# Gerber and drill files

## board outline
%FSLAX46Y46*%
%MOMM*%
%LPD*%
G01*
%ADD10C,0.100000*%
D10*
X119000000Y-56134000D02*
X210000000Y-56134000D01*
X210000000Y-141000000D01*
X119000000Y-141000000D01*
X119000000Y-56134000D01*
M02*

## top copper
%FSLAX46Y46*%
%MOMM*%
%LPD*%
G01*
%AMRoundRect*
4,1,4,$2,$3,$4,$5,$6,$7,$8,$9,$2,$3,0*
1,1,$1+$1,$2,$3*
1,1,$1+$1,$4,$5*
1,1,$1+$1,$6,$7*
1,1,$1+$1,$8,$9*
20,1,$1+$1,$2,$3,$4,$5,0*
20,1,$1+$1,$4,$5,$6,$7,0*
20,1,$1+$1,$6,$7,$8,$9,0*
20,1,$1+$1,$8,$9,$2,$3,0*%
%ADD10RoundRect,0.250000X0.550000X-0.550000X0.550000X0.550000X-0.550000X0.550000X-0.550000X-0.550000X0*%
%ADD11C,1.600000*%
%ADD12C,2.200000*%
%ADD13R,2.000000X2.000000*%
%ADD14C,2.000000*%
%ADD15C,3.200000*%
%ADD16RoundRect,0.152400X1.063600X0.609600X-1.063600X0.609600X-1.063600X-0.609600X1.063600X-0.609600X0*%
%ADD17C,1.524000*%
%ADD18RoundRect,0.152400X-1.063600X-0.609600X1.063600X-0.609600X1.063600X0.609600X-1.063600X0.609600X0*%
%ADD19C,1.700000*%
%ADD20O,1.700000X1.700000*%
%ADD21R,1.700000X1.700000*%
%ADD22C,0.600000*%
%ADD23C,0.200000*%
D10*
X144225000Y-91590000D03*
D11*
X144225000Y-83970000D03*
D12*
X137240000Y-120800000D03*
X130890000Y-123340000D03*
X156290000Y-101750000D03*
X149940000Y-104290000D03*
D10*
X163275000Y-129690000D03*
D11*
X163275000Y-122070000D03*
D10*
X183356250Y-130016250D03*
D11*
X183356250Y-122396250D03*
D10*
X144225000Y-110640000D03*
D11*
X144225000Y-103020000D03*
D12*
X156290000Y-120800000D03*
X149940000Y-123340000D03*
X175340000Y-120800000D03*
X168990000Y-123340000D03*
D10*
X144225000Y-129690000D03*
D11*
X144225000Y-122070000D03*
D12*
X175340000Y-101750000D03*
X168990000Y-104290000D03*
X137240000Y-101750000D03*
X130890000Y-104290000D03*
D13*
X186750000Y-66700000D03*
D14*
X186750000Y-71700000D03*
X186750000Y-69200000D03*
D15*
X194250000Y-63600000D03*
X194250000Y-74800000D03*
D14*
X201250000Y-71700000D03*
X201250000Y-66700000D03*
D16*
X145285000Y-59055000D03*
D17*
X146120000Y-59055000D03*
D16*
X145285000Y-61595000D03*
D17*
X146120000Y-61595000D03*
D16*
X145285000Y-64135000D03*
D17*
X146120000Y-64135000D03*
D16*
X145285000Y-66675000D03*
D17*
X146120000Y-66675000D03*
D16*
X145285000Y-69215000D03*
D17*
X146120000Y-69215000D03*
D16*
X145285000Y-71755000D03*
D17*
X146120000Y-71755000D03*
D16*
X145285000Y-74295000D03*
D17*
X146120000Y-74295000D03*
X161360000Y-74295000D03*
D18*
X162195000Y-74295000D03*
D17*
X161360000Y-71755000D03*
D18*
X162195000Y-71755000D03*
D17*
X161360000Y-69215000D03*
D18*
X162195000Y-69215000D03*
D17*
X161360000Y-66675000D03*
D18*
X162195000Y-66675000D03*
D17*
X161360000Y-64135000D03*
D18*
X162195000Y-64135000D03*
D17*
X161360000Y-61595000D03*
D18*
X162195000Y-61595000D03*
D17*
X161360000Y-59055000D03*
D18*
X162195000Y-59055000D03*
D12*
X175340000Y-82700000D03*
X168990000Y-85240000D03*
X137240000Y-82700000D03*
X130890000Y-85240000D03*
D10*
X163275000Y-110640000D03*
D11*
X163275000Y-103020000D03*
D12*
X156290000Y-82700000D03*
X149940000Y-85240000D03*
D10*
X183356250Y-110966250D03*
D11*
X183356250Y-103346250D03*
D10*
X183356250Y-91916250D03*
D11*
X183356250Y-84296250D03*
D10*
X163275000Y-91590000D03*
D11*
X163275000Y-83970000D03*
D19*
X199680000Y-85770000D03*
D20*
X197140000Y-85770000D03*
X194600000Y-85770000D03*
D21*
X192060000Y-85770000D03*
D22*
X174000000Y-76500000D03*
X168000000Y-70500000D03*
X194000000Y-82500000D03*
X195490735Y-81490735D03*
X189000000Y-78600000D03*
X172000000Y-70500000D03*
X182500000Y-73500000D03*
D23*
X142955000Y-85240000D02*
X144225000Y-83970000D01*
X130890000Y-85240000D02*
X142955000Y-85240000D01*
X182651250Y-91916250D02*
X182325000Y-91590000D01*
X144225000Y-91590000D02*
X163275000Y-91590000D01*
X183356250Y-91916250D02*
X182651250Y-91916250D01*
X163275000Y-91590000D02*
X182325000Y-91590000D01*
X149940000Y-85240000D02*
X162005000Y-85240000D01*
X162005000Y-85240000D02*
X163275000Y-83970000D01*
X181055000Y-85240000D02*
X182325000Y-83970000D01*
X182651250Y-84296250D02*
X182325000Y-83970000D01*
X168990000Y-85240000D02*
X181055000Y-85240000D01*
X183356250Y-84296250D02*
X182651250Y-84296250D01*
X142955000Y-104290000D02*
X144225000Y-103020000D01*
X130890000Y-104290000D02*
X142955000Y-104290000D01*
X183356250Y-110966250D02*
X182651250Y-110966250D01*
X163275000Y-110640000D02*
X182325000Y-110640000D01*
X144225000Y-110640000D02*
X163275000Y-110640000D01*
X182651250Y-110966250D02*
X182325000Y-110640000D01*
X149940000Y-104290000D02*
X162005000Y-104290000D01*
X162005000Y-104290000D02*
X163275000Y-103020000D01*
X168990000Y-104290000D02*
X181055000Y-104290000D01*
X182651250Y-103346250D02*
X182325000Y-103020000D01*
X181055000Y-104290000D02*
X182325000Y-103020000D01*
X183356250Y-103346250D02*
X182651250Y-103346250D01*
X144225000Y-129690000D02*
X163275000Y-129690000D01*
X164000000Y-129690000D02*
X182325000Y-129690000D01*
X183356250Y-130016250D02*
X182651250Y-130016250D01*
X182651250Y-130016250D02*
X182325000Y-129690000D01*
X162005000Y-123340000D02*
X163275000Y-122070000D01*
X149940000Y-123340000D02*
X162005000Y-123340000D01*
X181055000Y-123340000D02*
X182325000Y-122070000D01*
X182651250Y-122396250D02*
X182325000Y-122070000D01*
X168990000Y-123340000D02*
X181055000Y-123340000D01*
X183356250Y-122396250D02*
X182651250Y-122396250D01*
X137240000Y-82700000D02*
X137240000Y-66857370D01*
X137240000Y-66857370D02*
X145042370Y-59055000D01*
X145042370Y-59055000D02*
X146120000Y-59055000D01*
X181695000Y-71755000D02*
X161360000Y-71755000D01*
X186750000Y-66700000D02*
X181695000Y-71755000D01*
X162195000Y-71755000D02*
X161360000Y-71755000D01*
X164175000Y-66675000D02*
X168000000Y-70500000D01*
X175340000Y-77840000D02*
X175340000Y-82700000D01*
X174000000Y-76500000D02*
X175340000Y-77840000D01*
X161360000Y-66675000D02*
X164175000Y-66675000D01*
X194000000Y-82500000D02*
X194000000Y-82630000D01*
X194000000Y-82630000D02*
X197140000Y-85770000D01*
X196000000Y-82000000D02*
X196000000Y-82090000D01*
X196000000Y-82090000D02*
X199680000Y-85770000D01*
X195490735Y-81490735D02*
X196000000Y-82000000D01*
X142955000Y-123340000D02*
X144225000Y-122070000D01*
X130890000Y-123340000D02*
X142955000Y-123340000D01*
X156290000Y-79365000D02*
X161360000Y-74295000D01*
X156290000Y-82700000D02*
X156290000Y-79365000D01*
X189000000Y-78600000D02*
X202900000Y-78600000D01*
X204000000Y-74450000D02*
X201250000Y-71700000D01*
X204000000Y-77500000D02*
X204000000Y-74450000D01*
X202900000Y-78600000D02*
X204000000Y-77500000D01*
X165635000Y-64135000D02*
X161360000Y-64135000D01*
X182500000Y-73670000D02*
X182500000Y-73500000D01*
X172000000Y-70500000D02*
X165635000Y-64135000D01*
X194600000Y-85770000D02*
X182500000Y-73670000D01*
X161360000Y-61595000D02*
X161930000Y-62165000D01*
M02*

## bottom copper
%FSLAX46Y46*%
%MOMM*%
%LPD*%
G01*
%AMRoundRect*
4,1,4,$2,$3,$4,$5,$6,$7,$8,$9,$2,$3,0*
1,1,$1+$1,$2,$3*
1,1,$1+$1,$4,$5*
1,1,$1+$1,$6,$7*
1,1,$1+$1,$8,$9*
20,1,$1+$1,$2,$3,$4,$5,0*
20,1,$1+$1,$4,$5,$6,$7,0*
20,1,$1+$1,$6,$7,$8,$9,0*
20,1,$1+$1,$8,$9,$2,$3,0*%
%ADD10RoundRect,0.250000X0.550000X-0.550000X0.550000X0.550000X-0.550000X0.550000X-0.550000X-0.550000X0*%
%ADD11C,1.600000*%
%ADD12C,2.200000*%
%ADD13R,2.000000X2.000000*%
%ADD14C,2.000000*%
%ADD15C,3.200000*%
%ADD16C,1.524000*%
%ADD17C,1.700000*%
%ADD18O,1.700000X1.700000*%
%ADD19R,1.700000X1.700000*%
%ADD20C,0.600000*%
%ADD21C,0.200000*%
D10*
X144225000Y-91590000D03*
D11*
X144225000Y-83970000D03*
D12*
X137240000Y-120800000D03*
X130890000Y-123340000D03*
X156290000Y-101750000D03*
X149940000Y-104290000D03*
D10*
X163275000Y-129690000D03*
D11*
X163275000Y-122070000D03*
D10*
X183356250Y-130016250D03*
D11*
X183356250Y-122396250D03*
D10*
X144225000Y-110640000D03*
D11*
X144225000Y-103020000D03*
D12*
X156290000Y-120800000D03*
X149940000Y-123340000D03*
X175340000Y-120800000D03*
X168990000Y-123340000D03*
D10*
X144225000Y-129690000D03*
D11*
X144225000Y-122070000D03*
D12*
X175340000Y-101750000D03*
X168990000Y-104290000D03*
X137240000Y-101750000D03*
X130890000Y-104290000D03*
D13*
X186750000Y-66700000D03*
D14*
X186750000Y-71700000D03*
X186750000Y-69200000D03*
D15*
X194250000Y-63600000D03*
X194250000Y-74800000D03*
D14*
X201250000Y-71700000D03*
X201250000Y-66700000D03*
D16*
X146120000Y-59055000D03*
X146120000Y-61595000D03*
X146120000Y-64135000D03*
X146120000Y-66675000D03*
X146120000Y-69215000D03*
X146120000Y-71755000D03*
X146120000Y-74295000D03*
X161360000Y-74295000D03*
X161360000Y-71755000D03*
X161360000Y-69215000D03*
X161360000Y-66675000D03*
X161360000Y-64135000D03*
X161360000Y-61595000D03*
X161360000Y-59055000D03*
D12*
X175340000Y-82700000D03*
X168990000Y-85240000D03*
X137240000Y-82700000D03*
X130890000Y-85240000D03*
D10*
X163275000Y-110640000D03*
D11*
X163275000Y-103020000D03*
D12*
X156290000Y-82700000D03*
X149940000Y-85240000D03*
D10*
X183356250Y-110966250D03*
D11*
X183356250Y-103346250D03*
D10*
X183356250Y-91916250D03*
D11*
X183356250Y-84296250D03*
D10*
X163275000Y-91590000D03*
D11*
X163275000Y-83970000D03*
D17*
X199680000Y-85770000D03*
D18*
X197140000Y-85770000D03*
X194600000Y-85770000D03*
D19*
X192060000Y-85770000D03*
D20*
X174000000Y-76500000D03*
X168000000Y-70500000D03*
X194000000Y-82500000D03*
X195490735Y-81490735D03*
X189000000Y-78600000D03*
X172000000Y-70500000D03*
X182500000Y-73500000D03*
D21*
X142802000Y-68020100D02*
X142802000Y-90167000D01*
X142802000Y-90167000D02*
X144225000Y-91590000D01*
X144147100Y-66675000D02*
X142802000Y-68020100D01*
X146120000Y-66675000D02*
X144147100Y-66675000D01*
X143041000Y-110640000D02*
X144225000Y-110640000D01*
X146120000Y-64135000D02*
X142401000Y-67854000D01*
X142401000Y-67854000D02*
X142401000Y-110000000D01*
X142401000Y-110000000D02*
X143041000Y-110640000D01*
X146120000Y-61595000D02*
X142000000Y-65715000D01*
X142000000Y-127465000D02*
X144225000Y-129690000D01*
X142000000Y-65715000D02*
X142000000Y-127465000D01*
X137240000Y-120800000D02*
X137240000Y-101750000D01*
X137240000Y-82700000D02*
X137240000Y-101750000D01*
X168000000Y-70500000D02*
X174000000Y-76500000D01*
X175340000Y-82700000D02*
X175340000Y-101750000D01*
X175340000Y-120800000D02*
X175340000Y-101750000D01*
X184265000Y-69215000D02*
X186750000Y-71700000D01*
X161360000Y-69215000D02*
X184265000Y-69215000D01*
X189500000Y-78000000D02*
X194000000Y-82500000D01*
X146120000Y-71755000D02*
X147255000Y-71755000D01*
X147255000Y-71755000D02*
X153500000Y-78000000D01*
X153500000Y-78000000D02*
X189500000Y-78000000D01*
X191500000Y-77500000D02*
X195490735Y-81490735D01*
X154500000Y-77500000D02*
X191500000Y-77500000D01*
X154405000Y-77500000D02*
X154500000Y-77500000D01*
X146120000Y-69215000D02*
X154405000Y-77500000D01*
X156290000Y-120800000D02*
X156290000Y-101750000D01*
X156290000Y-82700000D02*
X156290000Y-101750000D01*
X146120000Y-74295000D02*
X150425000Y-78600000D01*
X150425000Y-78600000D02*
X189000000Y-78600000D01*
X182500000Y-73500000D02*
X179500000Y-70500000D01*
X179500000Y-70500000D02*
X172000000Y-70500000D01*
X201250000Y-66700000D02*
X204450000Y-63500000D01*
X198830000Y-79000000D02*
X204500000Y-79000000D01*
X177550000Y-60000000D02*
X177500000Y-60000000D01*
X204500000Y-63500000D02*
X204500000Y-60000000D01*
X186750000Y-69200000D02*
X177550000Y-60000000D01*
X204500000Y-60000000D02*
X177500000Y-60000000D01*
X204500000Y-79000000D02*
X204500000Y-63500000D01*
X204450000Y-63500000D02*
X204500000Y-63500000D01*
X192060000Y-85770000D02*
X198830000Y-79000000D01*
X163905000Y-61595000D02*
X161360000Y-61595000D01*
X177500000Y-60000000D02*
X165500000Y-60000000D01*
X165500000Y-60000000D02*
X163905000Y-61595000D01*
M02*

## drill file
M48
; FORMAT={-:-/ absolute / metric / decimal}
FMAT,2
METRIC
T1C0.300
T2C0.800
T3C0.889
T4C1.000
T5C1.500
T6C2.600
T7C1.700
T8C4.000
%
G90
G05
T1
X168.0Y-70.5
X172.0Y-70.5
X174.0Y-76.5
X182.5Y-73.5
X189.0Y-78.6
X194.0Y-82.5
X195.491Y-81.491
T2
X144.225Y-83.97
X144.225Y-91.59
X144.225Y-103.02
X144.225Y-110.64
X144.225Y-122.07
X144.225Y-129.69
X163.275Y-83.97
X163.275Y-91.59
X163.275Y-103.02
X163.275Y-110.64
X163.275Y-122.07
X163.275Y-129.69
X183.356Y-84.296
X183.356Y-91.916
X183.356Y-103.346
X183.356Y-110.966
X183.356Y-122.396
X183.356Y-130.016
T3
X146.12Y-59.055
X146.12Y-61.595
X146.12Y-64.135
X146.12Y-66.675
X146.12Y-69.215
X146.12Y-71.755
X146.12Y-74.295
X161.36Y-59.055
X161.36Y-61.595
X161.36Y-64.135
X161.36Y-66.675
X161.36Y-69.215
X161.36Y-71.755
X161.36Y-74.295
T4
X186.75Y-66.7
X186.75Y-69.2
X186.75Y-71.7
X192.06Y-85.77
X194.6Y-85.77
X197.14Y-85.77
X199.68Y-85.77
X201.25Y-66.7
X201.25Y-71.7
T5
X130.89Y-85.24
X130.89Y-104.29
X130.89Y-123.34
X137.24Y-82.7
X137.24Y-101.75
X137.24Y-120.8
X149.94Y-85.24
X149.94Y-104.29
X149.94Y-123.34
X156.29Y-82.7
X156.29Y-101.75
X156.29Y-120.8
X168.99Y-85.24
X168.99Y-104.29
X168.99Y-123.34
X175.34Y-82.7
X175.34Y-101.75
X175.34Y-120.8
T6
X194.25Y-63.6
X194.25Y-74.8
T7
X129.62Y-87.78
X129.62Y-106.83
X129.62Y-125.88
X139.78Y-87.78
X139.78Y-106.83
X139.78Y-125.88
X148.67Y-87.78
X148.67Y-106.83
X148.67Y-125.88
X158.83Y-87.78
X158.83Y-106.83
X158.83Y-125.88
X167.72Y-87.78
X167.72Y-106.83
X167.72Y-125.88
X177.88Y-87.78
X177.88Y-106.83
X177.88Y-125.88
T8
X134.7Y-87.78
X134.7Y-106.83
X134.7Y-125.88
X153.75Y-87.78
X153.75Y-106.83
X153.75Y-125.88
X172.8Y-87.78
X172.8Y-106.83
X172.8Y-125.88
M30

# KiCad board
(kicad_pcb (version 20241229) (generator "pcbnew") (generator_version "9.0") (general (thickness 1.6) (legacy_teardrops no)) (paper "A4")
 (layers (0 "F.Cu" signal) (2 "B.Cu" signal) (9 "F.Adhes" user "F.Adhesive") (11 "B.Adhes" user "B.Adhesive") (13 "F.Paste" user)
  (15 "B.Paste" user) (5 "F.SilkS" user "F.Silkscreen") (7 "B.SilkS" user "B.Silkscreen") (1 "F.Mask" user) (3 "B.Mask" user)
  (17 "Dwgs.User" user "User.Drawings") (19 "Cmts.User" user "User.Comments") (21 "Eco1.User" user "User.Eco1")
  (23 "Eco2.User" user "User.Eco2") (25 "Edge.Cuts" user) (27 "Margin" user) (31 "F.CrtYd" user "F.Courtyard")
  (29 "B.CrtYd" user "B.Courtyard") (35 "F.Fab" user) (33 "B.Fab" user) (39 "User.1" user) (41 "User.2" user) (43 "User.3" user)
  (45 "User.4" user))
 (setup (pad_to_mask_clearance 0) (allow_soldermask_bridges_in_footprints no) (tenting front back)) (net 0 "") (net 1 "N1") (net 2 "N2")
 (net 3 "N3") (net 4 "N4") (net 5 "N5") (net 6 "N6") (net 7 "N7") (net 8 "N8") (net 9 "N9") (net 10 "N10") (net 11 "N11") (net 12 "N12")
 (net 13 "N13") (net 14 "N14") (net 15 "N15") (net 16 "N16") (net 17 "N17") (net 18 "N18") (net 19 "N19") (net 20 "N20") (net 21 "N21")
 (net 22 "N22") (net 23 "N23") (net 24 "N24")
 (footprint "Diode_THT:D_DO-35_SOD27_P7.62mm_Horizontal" (layer "F.Cu") (at 144.225 91.59 90)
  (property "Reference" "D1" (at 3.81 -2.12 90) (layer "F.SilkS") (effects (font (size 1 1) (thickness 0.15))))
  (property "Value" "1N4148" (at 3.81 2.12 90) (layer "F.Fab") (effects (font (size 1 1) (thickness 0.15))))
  (pad "1" thru_hole roundrect (at 0 0 90) (size 1.6 1.6) (drill 0.8) (layers "*.Cu" "*.Mask") (remove_unused_layers no)
   (roundrect_rratio 0.15625) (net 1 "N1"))
  (pad "2" thru_hole circle (at 7.62 0 90) (size 1.6 1.6) (drill 0.8) (layers "*.Cu" "*.Mask") (remove_unused_layers no) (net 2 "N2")))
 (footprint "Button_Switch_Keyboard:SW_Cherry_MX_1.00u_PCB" (layer "F.Cu") (at 137.24 120.8)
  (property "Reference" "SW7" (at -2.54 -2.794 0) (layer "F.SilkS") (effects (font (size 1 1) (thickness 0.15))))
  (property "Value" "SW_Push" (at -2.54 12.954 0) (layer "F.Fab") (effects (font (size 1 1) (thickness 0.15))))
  (pad "" np_thru_hole circle (at -7.62 5.08) (size 1.7 1.7) (drill 1.7) (layers "*.Cu" "*.Mask"))
  (pad "" np_thru_hole circle (at -2.54 5.08) (size 4 4) (drill 4) (layers "*.Cu" "*.Mask"))
  (pad "" np_thru_hole circle (at 2.54 5.08) (size 1.7 1.7) (drill 1.7) (layers "*.Cu" "*.Mask"))
  (pad "1" thru_hole circle (at 0 0) (size 2.2 2.2) (drill 1.5) (layers "*.Cu" "*.Mask") (remove_unused_layers no) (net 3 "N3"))
  (pad "2" thru_hole circle (at -6.35 2.54) (size 2.2 2.2) (drill 1.5) (layers "*.Cu" "*.Mask") (remove_unused_layers no) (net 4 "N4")))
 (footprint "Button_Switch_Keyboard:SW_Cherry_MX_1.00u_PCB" (layer "F.Cu") (at 156.29 101.75)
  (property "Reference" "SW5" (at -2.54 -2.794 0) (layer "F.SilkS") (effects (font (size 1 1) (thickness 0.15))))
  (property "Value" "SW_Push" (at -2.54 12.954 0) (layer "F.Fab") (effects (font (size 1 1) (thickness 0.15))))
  (pad "" np_thru_hole circle (at -7.62 5.08) (size 1.7 1.7) (drill 1.7) (layers "*.Cu" "*.Mask"))
  (pad "" np_thru_hole circle (at -2.54 5.08) (size 4 4) (drill 4) (layers "*.Cu" "*.Mask"))
  (pad "" np_thru_hole circle (at 2.54 5.08) (size 1.7 1.7) (drill 1.7) (layers "*.Cu" "*.Mask"))
  (pad "1" thru_hole circle (at 0 0) (size 2.2 2.2) (drill 1.5) (layers "*.Cu" "*.Mask") (remove_unused_layers no) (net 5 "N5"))
  (pad "2" thru_hole circle (at -6.35 2.54) (size 2.2 2.2) (drill 1.5) (layers "*.Cu" "*.Mask") (remove_unused_layers no) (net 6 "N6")))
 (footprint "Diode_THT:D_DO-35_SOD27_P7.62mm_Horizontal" (layer "F.Cu") (at 163.275 129.69 90)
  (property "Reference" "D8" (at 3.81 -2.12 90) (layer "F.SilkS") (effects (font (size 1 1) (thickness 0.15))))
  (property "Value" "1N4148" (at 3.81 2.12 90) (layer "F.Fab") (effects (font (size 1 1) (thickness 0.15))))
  (pad "1" thru_hole roundrect (at 0 0 90) (size 1.6 1.6) (drill 0.8) (layers "*.Cu" "*.Mask") (remove_unused_layers no)
   (roundrect_rratio 0.15625) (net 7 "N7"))
  (pad "2" thru_hole circle (at 7.62 0 90) (size 1.6 1.6) (drill 0.8) (layers "*.Cu" "*.Mask") (remove_unused_layers no) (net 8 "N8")))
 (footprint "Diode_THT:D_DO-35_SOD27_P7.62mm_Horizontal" (layer "F.Cu") (at 183.35625 130.01625 90)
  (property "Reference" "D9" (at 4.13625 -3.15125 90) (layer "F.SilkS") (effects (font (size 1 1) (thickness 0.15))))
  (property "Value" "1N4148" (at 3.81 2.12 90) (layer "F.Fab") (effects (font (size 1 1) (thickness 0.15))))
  (pad "1" thru_hole roundrect (at 0 0 90) (size 1.6 1.6) (drill 0.8) (layers "*.Cu" "*.Mask") (remove_unused_layers no)
   (roundrect_rratio 0.15625) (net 7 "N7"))
  (pad "2" thru_hole circle (at 7.62 0 90) (size 1.6 1.6) (drill 0.8) (layers "*.Cu" "*.Mask") (remove_unused_layers no) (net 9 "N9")))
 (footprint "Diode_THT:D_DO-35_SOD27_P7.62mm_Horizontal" (layer "F.Cu") (at 144.225 110.64 90)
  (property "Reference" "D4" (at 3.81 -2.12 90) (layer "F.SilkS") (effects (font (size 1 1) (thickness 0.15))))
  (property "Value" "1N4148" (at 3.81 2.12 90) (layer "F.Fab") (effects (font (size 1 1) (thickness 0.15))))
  (pad "1" thru_hole roundrect (at 0 0 90) (size 1.6 1.6) (drill 0.8) (layers "*.Cu" "*.Mask") (remove_unused_layers no)
   (roundrect_rratio 0.15625) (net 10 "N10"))
  (pad "2" thru_hole circle (at 7.62 0 90) (size 1.6 1.6) (drill 0.8) (layers "*.Cu" "*.Mask") (remove_unused_layers no) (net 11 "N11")))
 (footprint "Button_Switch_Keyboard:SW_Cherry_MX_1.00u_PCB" (layer "F.Cu") (at 156.29 120.8)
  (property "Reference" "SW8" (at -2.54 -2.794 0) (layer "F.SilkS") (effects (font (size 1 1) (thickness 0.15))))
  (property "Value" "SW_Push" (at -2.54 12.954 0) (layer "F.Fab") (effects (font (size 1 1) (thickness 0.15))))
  (pad "" np_thru_hole circle (at -7.62 5.08) (size 1.7 1.7) (drill 1.7) (layers "*.Cu" "*.Mask"))
  (pad "" np_thru_hole circle (at -2.54 5.08) (size 4 4) (drill 4) (layers "*.Cu" "*.Mask"))
  (pad "" np_thru_hole circle (at 2.54 5.08) (size 1.7 1.7) (drill 1.7) (layers "*.Cu" "*.Mask"))
  (pad "1" thru_hole circle (at 0 0) (size 2.2 2.2) (drill 1.5) (layers "*.Cu" "*.Mask") (remove_unused_layers no) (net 5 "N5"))
  (pad "2" thru_hole circle (at -6.35 2.54) (size 2.2 2.2) (drill 1.5) (layers "*.Cu" "*.Mask") (remove_unused_layers no) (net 8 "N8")))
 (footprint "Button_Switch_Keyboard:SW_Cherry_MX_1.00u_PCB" (layer "F.Cu") (at 175.34 120.8)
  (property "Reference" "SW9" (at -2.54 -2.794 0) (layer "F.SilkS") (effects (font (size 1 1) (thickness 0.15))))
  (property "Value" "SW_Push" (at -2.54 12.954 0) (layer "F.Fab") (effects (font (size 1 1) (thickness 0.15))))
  (pad "" np_thru_hole circle (at -7.62 5.08) (size 1.7 1.7) (drill 1.7) (layers "*.Cu" "*.Mask"))
  (pad "" np_thru_hole circle (at -2.54 5.08) (size 4 4) (drill 4) (layers "*.Cu" "*.Mask"))
  (pad "" np_thru_hole circle (at 2.54 5.08) (size 1.7 1.7) (drill 1.7) (layers "*.Cu" "*.Mask"))
  (pad "1" thru_hole circle (at 0 0) (size 2.2 2.2) (drill 1.5) (layers "*.Cu" "*.Mask") (remove_unused_layers no) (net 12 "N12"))
  (pad "2" thru_hole circle (at -6.35 2.54) (size 2.2 2.2) (drill 1.5) (layers "*.Cu" "*.Mask") (remove_unused_layers no) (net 9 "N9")))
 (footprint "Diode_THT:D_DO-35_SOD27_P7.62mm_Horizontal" (layer "F.Cu") (at 144.225 129.69 90)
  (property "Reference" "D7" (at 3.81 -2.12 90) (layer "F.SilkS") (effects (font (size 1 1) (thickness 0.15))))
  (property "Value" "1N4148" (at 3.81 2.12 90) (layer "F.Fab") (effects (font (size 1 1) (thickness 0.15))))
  (pad "1" thru_hole roundrect (at 0 0 90) (size 1.6 1.6) (drill 0.8) (layers "*.Cu" "*.Mask") (remove_unused_layers no)
   (roundrect_rratio 0.15625) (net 7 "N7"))
  (pad "2" thru_hole circle (at 7.62 0 90) (size 1.6 1.6) (drill 0.8) (layers "*.Cu" "*.Mask") (remove_unused_layers no) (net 4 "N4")))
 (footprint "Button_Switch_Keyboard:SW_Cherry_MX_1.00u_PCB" (layer "F.Cu") (at 175.34 101.75)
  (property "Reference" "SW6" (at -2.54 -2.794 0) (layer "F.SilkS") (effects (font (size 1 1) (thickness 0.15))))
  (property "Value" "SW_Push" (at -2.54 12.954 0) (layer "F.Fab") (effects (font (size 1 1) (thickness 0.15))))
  (pad "" np_thru_hole circle (at -7.62 5.08) (size 1.7 1.7) (drill 1.7) (layers "*.Cu" "*.Mask"))
  (pad "" np_thru_hole circle (at -2.54 5.08) (size 4 4) (drill 4) (layers "*.Cu" "*.Mask"))
  (pad "" np_thru_hole circle (at 2.54 5.08) (size 1.7 1.7) (drill 1.7) (layers "*.Cu" "*.Mask"))
  (pad "1" thru_hole circle (at 0 0) (size 2.2 2.2) (drill 1.5) (layers "*.Cu" "*.Mask") (remove_unused_layers no) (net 12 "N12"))
  (pad "2" thru_hole circle (at -6.35 2.54) (size 2.2 2.2) (drill 1.5) (layers "*.Cu" "*.Mask") (remove_unused_layers no) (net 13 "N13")))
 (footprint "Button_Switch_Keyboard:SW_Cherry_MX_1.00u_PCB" (layer "F.Cu") (at 137.24 101.75)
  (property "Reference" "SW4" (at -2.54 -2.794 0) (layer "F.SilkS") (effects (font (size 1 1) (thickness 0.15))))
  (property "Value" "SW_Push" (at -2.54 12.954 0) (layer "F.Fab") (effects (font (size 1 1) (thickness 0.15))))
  (pad "" np_thru_hole circle (at -7.62 5.08) (size 1.7 1.7) (drill 1.7) (layers "*.Cu" "*.Mask"))
  (pad "" np_thru_hole circle (at -2.54 5.08) (size 4 4) (drill 4) (layers "*.Cu" "*.Mask"))
  (pad "" np_thru_hole circle (at 2.54 5.08) (size 1.7 1.7) (drill 1.7) (layers "*.Cu" "*.Mask"))
  (pad "1" thru_hole circle (at 0 0) (size 2.2 2.2) (drill 1.5) (layers "*.Cu" "*.Mask") (remove_unused_layers no) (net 3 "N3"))
  (pad "2" thru_hole circle (at -6.35 2.54) (size 2.2 2.2) (drill 1.5) (layers "*.Cu" "*.Mask") (remove_unused_layers no) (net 11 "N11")))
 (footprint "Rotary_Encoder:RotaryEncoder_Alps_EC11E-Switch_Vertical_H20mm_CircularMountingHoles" (layer "F.Cu") (at 186.75 66.7)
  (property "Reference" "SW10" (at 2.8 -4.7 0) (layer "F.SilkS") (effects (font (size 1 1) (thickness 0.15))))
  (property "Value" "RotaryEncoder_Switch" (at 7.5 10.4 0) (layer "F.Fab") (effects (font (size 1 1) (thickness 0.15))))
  (pad "A" thru_hole rect (at 0 0) (size 2 2) (drill 1) (layers "*.Cu" "*.Mask") (remove_unused_layers no) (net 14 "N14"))
  (pad "B" thru_hole circle (at 0 5) (size 2 2) (drill 1) (layers "*.Cu" "*.Mask") (remove_unused_layers no) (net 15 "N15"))
  (pad "C" thru_hole circle (at 0 2.5) (size 2 2) (drill 1) (layers "*.Cu" "*.Mask") (remove_unused_layers no) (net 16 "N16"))
  (pad "MP" thru_hole circle (at 7.5 -3.1) (size 3.2 3.2) (drill 2.6) (layers "*.Cu" "*.Mask") (remove_unused_layers no))
  (pad "MP" thru_hole circle (at 7.5 8.1) (size 3.2 3.2) (drill 2.6) (layers "*.Cu" "*.Mask") (remove_unused_layers no))
  (pad "S1" thru_hole circle (at 14.5 5) (size 2 2) (drill 1) (layers "*.Cu" "*.Mask") (remove_unused_layers no) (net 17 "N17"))
  (pad "S2" thru_hole circle (at 14.5 0) (size 2 2) (drill 1) (layers "*.Cu" "*.Mask") (remove_unused_layers no) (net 16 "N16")))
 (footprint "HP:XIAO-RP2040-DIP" (layer "F.Cu") (at 153.74 66.675)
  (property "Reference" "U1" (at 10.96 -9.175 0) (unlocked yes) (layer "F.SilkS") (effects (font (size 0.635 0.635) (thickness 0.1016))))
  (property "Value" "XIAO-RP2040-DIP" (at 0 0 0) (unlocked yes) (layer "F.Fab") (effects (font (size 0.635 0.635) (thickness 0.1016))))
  (pad "1" smd roundrect (at -8.455 -7.62 180) (size 2.432 1.524) (layers "F.Cu" "F.Mask") (roundrect_rratio 0.1) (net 3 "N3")
   (thermal_bridge_angle 45))
  (pad "1" thru_hole circle (at -7.62 -7.62 180) (size 1.524 1.524) (drill 0.889) (layers "*.Cu" "*.Mask") (remove_unused_layers no)
   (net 3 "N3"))
  (pad "2" smd roundrect (at -8.455 -5.08 180) (size 2.432 1.524) (layers "F.Cu" "F.Mask") (roundrect_rratio 0.1) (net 7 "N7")
   (thermal_bridge_angle 45))
  (pad "2" thru_hole circle (at -7.62 -5.08 180) (size 1.524 1.524) (drill 0.889) (layers "*.Cu" "*.Mask") (remove_unused_layers no)
   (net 7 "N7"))
  (pad "3" smd roundrect (at -8.455 -2.54 180) (size 2.432 1.524) (layers "F.Cu" "F.Mask") (roundrect_rratio 0.1) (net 10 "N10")
   (thermal_bridge_angle 45))
  (pad "3" thru_hole circle (at -7.62 -2.54 180) (size 1.524 1.524) (drill 0.889) (layers "*.Cu" "*.Mask") (remove_unused_layers no)
   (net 10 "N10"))
  (pad "4" smd roundrect (at -8.455 0 180) (size 2.432 1.524) (layers "F.Cu" "F.Mask") (roundrect_rratio 0.1) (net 1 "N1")
   (thermal_bridge_angle 45))
  (pad "4" thru_hole circle (at -7.62 0 180) (size 1.524 1.524) (drill 0.889) (layers "*.Cu" "*.Mask") (remove_unused_layers no)
   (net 1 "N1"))
  (pad "5" smd roundrect (at -8.455 2.54 180) (size 2.432 1.524) (layers "F.Cu" "F.Mask") (roundrect_rratio 0.1) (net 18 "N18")
   (thermal_bridge_angle 45))
  (pad "5" thru_hole circle (at -7.62 2.54 180) (size 1.524 1.524) (drill 0.889) (layers "*.Cu" "*.Mask") (remove_unused_layers no)
   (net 18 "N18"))
  (pad "6" smd roundrect (at -8.455 5.08 180) (size 2.432 1.524) (layers "F.Cu" "F.Mask") (roundrect_rratio 0.1) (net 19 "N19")
   (thermal_bridge_angle 45))
  (pad "6" thru_hole circle (at -7.62 5.08 180) (size 1.524 1.524) (drill 0.889) (layers "*.Cu" "*.Mask") (remove_unused_layers no)
   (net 19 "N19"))
  (pad "7" smd roundrect (at -8.455 7.62 180) (size 2.432 1.524) (layers "F.Cu" "F.Mask") (roundrect_rratio 0.1) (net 17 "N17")
   (thermal_bridge_angle 45))
  (pad "7" thru_hole circle (at -7.62 7.62 180) (size 1.524 1.524) (drill 0.889) (layers "*.Cu" "*.Mask") (remove_unused_layers no)
   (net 17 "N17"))
  (pad "8" thru_hole circle (at 7.62 7.62) (size 1.524 1.524) (drill 0.889) (layers "*.Cu" "*.Mask") (remove_unused_layers no) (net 5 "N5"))
  (pad "8" smd roundrect (at 8.455 7.62) (size 2.432 1.524) (layers "F.Cu" "F.Mask") (roundrect_rratio 0.1) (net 5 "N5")
   (thermal_bridge_angle 45))
  (pad "9" thru_hole circle (at 7.62 5.08) (size 1.524 1.524) (drill 0.889) (layers "*.Cu" "*.Mask") (remove_unused_layers no)
   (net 14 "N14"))
  (pad "9" smd roundrect (at 8.455 5.08) (size 2.432 1.524) (layers "F.Cu" "F.Mask") (roundrect_rratio 0.1) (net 14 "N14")
   (thermal_bridge_angle 45))
  (pad "10" thru_hole circle (at 7.62 2.54) (size 1.524 1.524) (drill 0.889) (layers "*.Cu" "*.Mask") (remove_unused_layers no)
   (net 15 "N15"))
  (pad "10" smd roundrect (at 8.455 2.54) (size 2.432 1.524) (layers "F.Cu" "F.Mask") (roundrect_rratio 0.1) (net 15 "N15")
   (thermal_bridge_angle 45))
  (pad "11" thru_hole circle (at 7.62 0) (size 1.524 1.524) (drill 0.889) (layers "*.Cu" "*.Mask") (remove_unused_layers no) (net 12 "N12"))
  (pad "11" smd roundrect (at 8.455 0) (size 2.432 1.524) (layers "F.Cu" "F.Mask") (roundrect_rratio 0.1) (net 12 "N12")
   (thermal_bridge_angle 45))
  (pad "12" thru_hole circle (at 7.62 -2.54) (size 1.524 1.524) (drill 0.889) (layers "*.Cu" "*.Mask") (remove_unused_layers no)
   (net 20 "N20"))
  (pad "12" smd roundrect (at 8.455 -2.54) (size 2.432 1.524) (layers "F.Cu" "F.Mask") (roundrect_rratio 0.1) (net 20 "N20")
   (thermal_bridge_angle 45))
  (pad "13" thru_hole circle (at 7.62 -5.08) (size 1.524 1.524) (drill 0.889) (layers "*.Cu" "*.Mask") (remove_unused_layers no)
   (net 16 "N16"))
  (pad "13" smd roundrect (at 8.455 -5.08) (size 2.432 1.524) (layers "F.Cu" "F.Mask") (roundrect_rratio 0.1) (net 16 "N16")
   (thermal_bridge_angle 45))
  (pad "14" thru_hole circle (at 7.62 -7.62) (size 1.524 1.524) (drill 0.889) (layers "*.Cu" "*.Mask") (remove_unused_layers no)
   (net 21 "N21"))
  (pad "14" smd roundrect (at 8.455 -7.62) (size 2.432 1.524) (layers "F.Cu" "F.Mask") (roundrect_rratio 0.1) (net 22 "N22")
   (thermal_bridge_angle 45)))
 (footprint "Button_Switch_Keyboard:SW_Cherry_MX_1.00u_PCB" (layer "F.Cu") (at 175.34 82.7)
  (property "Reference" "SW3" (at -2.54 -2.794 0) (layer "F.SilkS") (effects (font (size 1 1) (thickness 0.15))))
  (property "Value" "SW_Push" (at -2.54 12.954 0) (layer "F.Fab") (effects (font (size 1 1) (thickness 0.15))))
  (pad "" np_thru_hole circle (at -7.62 5.08) (size 1.7 1.7) (drill 1.7) (layers "*.Cu" "*.Mask"))
  (pad "" np_thru_hole circle (at -2.54 5.08) (size 4 4) (drill 4) (layers "*.Cu" "*.Mask"))
  (pad "" np_thru_hole circle (at 2.54 5.08) (size 1.7 1.7) (drill 1.7) (layers "*.Cu" "*.Mask"))
  (pad "1" thru_hole circle (at 0 0) (size 2.2 2.2) (drill 1.5) (layers "*.Cu" "*.Mask") (remove_unused_layers no) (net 12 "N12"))
  (pad "2" thru_hole circle (at -6.35 2.54) (size 2.2 2.2) (drill 1.5) (layers "*.Cu" "*.Mask") (remove_unused_layers no) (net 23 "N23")))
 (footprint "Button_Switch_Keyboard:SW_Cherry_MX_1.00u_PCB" (layer "F.Cu") (at 137.24 82.7)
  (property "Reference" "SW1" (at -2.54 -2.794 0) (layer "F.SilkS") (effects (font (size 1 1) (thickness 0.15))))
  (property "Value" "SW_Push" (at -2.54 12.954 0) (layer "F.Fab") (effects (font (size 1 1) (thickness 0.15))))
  (pad "" np_thru_hole circle (at -7.62 5.08) (size 1.7 1.7) (drill 1.7) (layers "*.Cu" "*.Mask"))
  (pad "" np_thru_hole circle (at -2.54 5.08) (size 4 4) (drill 4) (layers "*.Cu" "*.Mask"))
  (pad "" np_thru_hole circle (at 2.54 5.08) (size 1.7 1.7) (drill 1.7) (layers "*.Cu" "*.Mask"))
  (pad "1" thru_hole circle (at 0 0) (size 2.2 2.2) (drill 1.5) (layers "*.Cu" "*.Mask") (remove_unused_layers no) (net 3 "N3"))
  (pad "2" thru_hole circle (at -6.35 2.54) (size 2.2 2.2) (drill 1.5) (layers "*.Cu" "*.Mask") (remove_unused_layers no) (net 2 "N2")))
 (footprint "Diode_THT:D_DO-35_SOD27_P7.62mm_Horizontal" (layer "F.Cu") (at 163.275 110.64 90)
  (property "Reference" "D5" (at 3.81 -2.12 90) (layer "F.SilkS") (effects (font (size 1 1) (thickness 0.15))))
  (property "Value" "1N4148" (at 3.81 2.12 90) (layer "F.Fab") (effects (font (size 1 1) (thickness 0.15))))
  (pad "1" thru_hole roundrect (at 0 0 90) (size 1.6 1.6) (drill 0.8) (layers "*.Cu" "*.Mask") (remove_unused_layers no)
   (roundrect_rratio 0.15625) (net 10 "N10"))
  (pad "2" thru_hole circle (at 7.62 0 90) (size 1.6 1.6) (drill 0.8) (layers "*.Cu" "*.Mask") (remove_unused_layers no) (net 6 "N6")))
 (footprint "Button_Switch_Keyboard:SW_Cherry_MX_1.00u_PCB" (layer "F.Cu") (at 156.29 82.7)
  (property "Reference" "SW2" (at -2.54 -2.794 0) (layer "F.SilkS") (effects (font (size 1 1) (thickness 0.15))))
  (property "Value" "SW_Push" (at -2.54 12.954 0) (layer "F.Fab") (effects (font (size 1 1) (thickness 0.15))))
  (pad "" np_thru_hole circle (at -7.62 5.08) (size 1.7 1.7) (drill 1.7) (layers "*.Cu" "*.Mask"))
  (pad "" np_thru_hole circle (at -2.54 5.08) (size 4 4) (drill 4) (layers "*.Cu" "*.Mask"))
  (pad "" np_thru_hole circle (at 2.54 5.08) (size 1.7 1.7) (drill 1.7) (layers "*.Cu" "*.Mask"))
  (pad "1" thru_hole circle (at 0 0) (size 2.2 2.2) (drill 1.5) (layers "*.Cu" "*.Mask") (remove_unused_layers no) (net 5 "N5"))
  (pad "2" thru_hole circle (at -6.35 2.54) (size 2.2 2.2) (drill 1.5) (layers "*.Cu" "*.Mask") (remove_unused_layers no) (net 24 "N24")))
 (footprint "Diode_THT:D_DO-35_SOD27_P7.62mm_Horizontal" (layer "F.Cu") (at 183.35625 110.96625 90)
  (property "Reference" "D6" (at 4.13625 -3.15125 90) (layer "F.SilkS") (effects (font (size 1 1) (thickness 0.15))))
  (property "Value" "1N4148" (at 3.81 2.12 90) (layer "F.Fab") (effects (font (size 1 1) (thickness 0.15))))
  (pad "1" thru_hole roundrect (at 0 0 90) (size 1.6 1.6) (drill 0.8) (layers "*.Cu" "*.Mask") (remove_unused_layers no)
   (roundrect_rratio 0.15625) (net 10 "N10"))
  (pad "2" thru_hole circle (at 7.62 0 90) (size 1.6 1.6) (drill 0.8) (layers "*.Cu" "*.Mask") (remove_unused_layers no) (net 13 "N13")))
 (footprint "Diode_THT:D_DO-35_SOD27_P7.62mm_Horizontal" (layer "F.Cu") (at 183.35625 91.91625 90)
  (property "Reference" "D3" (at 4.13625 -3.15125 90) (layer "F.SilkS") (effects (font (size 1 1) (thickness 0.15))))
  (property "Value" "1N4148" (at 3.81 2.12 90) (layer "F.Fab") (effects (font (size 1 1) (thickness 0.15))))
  (pad "1" thru_hole roundrect (at 0 0 90) (size 1.6 1.6) (drill 0.8) (layers "*.Cu" "*.Mask") (remove_unused_layers no)
   (roundrect_rratio 0.15625) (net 1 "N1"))
  (pad "2" thru_hole circle (at 7.62 0 90) (size 1.6 1.6) (drill 0.8) (layers "*.Cu" "*.Mask") (remove_unused_layers no) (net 23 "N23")))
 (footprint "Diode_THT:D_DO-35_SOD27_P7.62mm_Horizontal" (layer "F.Cu") (at 163.275 91.59 90)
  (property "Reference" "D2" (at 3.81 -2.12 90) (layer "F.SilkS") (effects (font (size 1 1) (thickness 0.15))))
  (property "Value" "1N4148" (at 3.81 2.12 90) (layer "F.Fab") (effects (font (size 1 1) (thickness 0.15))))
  (pad "1" thru_hole roundrect (at 0 0 90) (size 1.6 1.6) (drill 0.8) (layers "*.Cu" "*.Mask") (remove_unused_layers no)
   (roundrect_rratio 0.15625) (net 1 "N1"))
  (pad "2" thru_hole circle (at 7.62 0 90) (size 1.6 1.6) (drill 0.8) (layers "*.Cu" "*.Mask") (remove_unused_layers no) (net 24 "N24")))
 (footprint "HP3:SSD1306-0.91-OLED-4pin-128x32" (layer "B.Cu") (at 201.87 122.27 90)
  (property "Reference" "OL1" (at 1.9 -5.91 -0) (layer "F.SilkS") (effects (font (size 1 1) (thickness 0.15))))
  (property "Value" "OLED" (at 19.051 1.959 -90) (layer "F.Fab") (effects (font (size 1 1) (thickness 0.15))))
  (pad "1" thru_hole circle (at 36.5 -2.19 90) (size 1.7 1.7) (drill 1) (layers "*.Cu" "*.Mask") (remove_unused_layers no) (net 18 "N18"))
  (pad "2" thru_hole oval (at 36.5 -4.73 90) (size 1.7 1.7) (drill 1) (layers "*.Cu" "*.Mask") (remove_unused_layers no) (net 19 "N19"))
  (pad "3" thru_hole oval (at 36.5 -7.27 90) (size 1.7 1.7) (drill 1) (layers "*.Cu" "*.Mask") (remove_unused_layers no) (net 20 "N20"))
  (pad "4" thru_hole rect (at 36.5 -9.81 90) (size 1.7 1.7) (drill 1) (layers "*.Cu" "*.Mask") (remove_unused_layers no) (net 16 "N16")))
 (gr_rect (start 119 56.134) (end 210 141) (stroke (width 0.1) (type solid)) (fill no) (layer "Edge.Cuts"))
 (segment (start 142.955 85.24) (end 144.225 83.97) (width 0.2) (layer "F.Cu") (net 2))
 (segment (start 130.89 85.24) (end 142.955 85.24) (width 0.2) (layer "F.Cu") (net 2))
 (segment (start 182.65125 91.91625) (end 182.325 91.59) (width 0.2) (layer "F.Cu") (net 1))
 (segment (start 144.225 91.59) (end 163.275 91.59) (width 0.2) (layer "F.Cu") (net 1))
 (segment (start 183.35625 91.91625) (end 182.65125 91.91625) (width 0.2) (layer "F.Cu") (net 1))
 (segment (start 163.275 91.59) (end 182.325 91.59) (width 0.2) (layer "F.Cu") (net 1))
 (segment (start 142.802 68.0201) (end 142.802 90.167) (width 0.2) (layer "B.Cu") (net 1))
 (segment (start 142.802 90.167) (end 144.225 91.59) (width 0.2) (layer "B.Cu") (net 1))
 (segment (start 144.1471 66.675) (end 142.802 68.0201) (width 0.2) (layer "B.Cu") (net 1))
 (segment (start 146.12 66.675) (end 144.1471 66.675) (width 0.2) (layer "B.Cu") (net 1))
 (segment (start 149.94 85.24) (end 162.005 85.24) (width 0.2) (layer "F.Cu") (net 24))
 (segment (start 162.005 85.24) (end 163.275 83.97) (width 0.2) (layer "F.Cu") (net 24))
 (segment (start 181.055 85.24) (end 182.325 83.97) (width 0.2) (layer "F.Cu") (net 23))
 (segment (start 182.65125 84.29625) (end 182.325 83.97) (width 0.2) (layer "F.Cu") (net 23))
 (segment (start 168.99 85.24) (end 181.055 85.24) (width 0.2) (layer "F.Cu") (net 23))
 (segment (start 183.35625 84.29625) (end 182.65125 84.29625) (width 0.2) (layer "F.Cu") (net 23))
 (segment (start 142.955 104.29) (end 144.225 103.02) (width 0.2) (layer "F.Cu") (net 11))
 (segment (start 130.89 104.29) (end 142.955 104.29) (width 0.2) (layer "F.Cu") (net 11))
 (segment (start 183.35625 110.96625) (end 182.65125 110.96625) (width 0.2) (layer "F.Cu") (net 10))
 (segment (start 163.275 110.64) (end 182.325 110.64) (width 0.2) (layer "F.Cu") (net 10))
 (segment (start 144.225 110.64) (end 163.275 110.64) (width 0.2) (layer "F.Cu") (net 10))
 (segment (start 182.65125 110.96625) (end 182.325 110.64) (width 0.2) (layer "F.Cu") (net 10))
 (segment (start 143.041 110.64) (end 144.225 110.64) (width 0.2) (layer "B.Cu") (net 10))
 (segment (start 146.12 64.135) (end 142.401 67.854) (width 0.2) (layer "B.Cu") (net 10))
 (segment (start 142.401 67.854) (end 142.401 110) (width 0.2) (layer "B.Cu") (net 10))
 (segment (start 142.401 110) (end 143.041 110.64) (width 0.2) (layer "B.Cu") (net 10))
 (segment (start 149.94 104.29) (end 162.005 104.29) (width 0.2) (layer "F.Cu") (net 6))
 (segment (start 162.005 104.29) (end 163.275 103.02) (width 0.2) (layer "F.Cu") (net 6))
 (segment (start 168.99 104.29) (end 181.055 104.29) (width 0.2) (layer "F.Cu") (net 13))
 (segment (start 182.65125 103.34625) (end 182.325 103.02) (width 0.2) (layer "F.Cu") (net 13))
 (segment (start 181.055 104.29) (end 182.325 103.02) (width 0.2) (layer "F.Cu") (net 13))
 (segment (start 183.35625 103.34625) (end 182.65125 103.34625) (width 0.2) (layer "F.Cu") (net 13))
 (segment (start 144.225 129.69) (end 163.275 129.69) (width 0.2) (layer "F.Cu") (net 7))
 (segment (start 164 129.69) (end 182.325 129.69) (width 0.2) (layer "F.Cu") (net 7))
 (segment (start 183.35625 130.01625) (end 182.65125 130.01625) (width 0.2) (layer "F.Cu") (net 7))
 (segment (start 182.65125 130.01625) (end 182.325 129.69) (width 0.2) (layer "F.Cu") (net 7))
 (segment (start 146.12 61.595) (end 142 65.715) (width 0.2) (layer "B.Cu") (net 7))
 (segment (start 142 127.465) (end 144.225 129.69) (width 0.2) (layer "B.Cu") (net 7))
 (segment (start 142 65.715) (end 142 127.465) (width 0.2) (layer "B.Cu") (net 7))
 (segment (start 162.005 123.34) (end 163.275 122.07) (width 0.2) (layer "F.Cu") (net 8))
 (segment (start 149.94 123.34) (end 162.005 123.34) (width 0.2) (layer "F.Cu") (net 8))
 (segment (start 181.055 123.34) (end 182.325 122.07) (width 0.2) (layer "F.Cu") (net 9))
 (segment (start 182.65125 122.39625) (end 182.325 122.07) (width 0.2) (layer "F.Cu") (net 9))
 (segment (start 168.99 123.34) (end 181.055 123.34) (width 0.2) (layer "F.Cu") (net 9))
 (segment (start 183.35625 122.39625) (end 182.65125 122.39625) (width 0.2) (layer "F.Cu") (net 9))
 (segment (start 137.24 82.7) (end 137.24 66.85737) (width 0.2) (layer "F.Cu") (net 3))
 (segment (start 137.24 66.85737) (end 145.04237 59.055) (width 0.2) (layer "F.Cu") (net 3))
 (segment (start 145.04237 59.055) (end 146.12 59.055) (width 0.2) (layer "F.Cu") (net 3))
 (segment (start 137.24 120.8) (end 137.24 101.75) (width 0.2) (layer "B.Cu") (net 3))
 (segment (start 137.24 82.7) (end 137.24 101.75) (width 0.2) (layer "B.Cu") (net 3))
 (segment (start 181.695 71.755) (end 161.36 71.755) (width 0.2) (layer "F.Cu") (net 14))
 (segment (start 186.75 66.7) (end 181.695 71.755) (width 0.2) (layer "F.Cu") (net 14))
 (segment (start 162.195 71.755) (end 161.36 71.755) (width 0.2) (layer "F.Cu") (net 14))
 (segment (start 164.175 66.675) (end 168 70.5) (width 0.2) (layer "F.Cu") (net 12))
 (segment (start 175.34 77.84) (end 175.34 82.7) (width 0.2) (layer "F.Cu") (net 12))
 (segment (start 174 76.5) (end 175.34 77.84) (width 0.2) (layer "F.Cu") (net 12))
 (segment (start 161.36 66.675) (end 164.175 66.675) (width 0.2) (layer "F.Cu") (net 12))
 (via (at 174 76.5) (size 0.6) (drill 0.3) (layers "F.Cu" "B.Cu") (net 12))
 (via (at 168 70.5) (size 0.6) (drill 0.3) (layers "F.Cu" "B.Cu") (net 12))
 (segment (start 168 70.5) (end 174 76.5) (width 0.2) (layer "B.Cu") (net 12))
 (segment (start 175.34 82.7) (end 175.34 101.75) (width 0.2) (layer "B.Cu") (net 12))
 (segment (start 175.34 120.8) (end 175.34 101.75) (width 0.2) (layer "B.Cu") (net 12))
 (segment (start 184.265 69.215) (end 186.75 71.7) (width 0.2) (layer "B.Cu") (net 15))
 (segment (start 161.36 69.215) (end 184.265 69.215) (width 0.2) (layer "B.Cu") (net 15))
 (segment (start 194 82.5) (end 194 82.63) (width 0.2) (layer "F.Cu") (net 19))
 (segment (start 194 82.63) (end 197.14 85.77) (width 0.2) (layer "F.Cu") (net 19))
 (via (at 194 82.5) (size 0.6) (drill 0.3) (layers "F.Cu" "B.Cu") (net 19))
 (segment (start 189.5 78) (end 194 82.5) (width 0.2) (layer "B.Cu") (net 19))
 (segment (start 146.12 71.755) (end 147.255 71.755) (width 0.2) (layer "B.Cu") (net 19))
 (segment (start 147.255 71.755) (end 153.5 78) (width 0.2) (layer "B.Cu") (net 19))
 (segment (start 153.5 78) (end 189.5 78) (width 0.2) (layer "B.Cu") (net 19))
 (segment (start 196 82) (end 196 82.09) (width 0.2) (layer "F.Cu") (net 18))
 (segment (start 196 82.09) (end 199.68 85.77) (width 0.2) (layer "F.Cu") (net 18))
 (segment (start 195.490735 81.490735) (end 196 82) (width 0.2) (layer "F.Cu") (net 18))
 (via (at 195.490735 81.490735) (size 0.6) (drill 0.3) (layers "F.Cu" "B.Cu") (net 18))
 (segment (start 191.5 77.5) (end 195.490735 81.490735) (width 0.2) (layer "B.Cu") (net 18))
 (segment (start 154.5 77.5) (end 191.5 77.5) (width 0.2) (layer "B.Cu") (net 18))
 (segment (start 154.405 77.5) (end 154.5 77.5) (width 0.2) (layer "B.Cu") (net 18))
 (segment (start 146.12 69.215) (end 154.405 77.5) (width 0.2) (layer "B.Cu") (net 18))
 (segment (start 142.955 123.34) (end 144.225 122.07) (width 0.2) (layer "F.Cu") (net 4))
 (segment (start 130.89 123.34) (end 142.955 123.34) (width 0.2) (layer "F.Cu") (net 4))
 (segment (start 156.29 79.365) (end 161.36 74.295) (width 0.2) (layer "F.Cu") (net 5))
 (segment (start 156.29 82.7) (end 156.29 79.365) (width 0.2) (layer "F.Cu") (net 5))
 (segment (start 156.29 120.8) (end 156.29 101.75) (width 0.2) (layer "B.Cu") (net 5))
 (segment (start 156.29 82.7) (end 156.29 101.75) (width 0.2) (layer "B.Cu") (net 5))
 (segment (start 189 78.6) (end 202.9 78.6) (width 0.2) (layer "F.Cu") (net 17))
 (segment (start 204 74.45) (end 201.25 71.7) (width 0.2) (layer "F.Cu") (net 17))
 (segment (start 204 77.5) (end 204 74.45) (width 0.2) (layer "F.Cu") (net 17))
 (segment (start 202.9 78.6) (end 204 77.5) (width 0.2) (layer "F.Cu") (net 17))
 (via (at 189 78.6) (size 0.6) (drill 0.3) (layers "F.Cu" "B.Cu") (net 17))
 (segment (start 146.12 74.295) (end 150.425 78.6) (width 0.2) (layer "B.Cu") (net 17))
 (segment (start 150.425 78.6) (end 189 78.6) (width 0.2) (layer "B.Cu") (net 17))
 (segment (start 165.635 64.135) (end 161.36 64.135) (width 0.2) (layer "F.Cu") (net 20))
 (segment (start 182.5 73.67) (end 182.5 73.5) (width 0.2) (layer "F.Cu") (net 20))
 (segment (start 172 70.5) (end 165.635 64.135) (width 0.2) (layer "F.Cu") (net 20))
 (segment (start 194.6 85.77) (end 182.5 73.67) (width 0.2) (layer "F.Cu") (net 20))
 (via (at 172 70.5) (size 0.6) (drill 0.3) (layers "F.Cu" "B.Cu") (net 20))
 (via (at 182.5 73.5) (size 0.6) (drill 0.3) (layers "F.Cu" "B.Cu") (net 20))
 (segment (start 182.5 73.5) (end 179.5 70.5) (width 0.2) (layer "B.Cu") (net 20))
 (segment (start 179.5 70.5) (end 172 70.5) (width 0.2) (layer "B.Cu") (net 20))
 (segment (start 161.36 61.595) (end 161.93 62.165) (width 0.2) (layer "F.Cu") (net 16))
 (segment (start 201.25 66.7) (end 204.45 63.5) (width 0.2) (layer "B.Cu") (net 16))
 (segment (start 198.83 79) (end 204.5 79) (width 0.2) (layer "B.Cu") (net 16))
 (segment (start 177.55 60) (end 177.5 60) (width 0.2) (layer "B.Cu") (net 16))
 (segment (start 204.5 63.5) (end 204.5 60) (width 0.2) (layer "B.Cu") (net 16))
 (segment (start 186.75 69.2) (end 177.55 60) (width 0.2) (layer "B.Cu") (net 16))
 (segment (start 204.5 60) (end 177.5 60) (width 0.2) (layer "B.Cu") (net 16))
 (segment (start 204.5 79) (end 204.5 63.5) (width 0.2) (layer "B.Cu") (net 16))
 (segment (start 204.45 63.5) (end 204.5 63.5) (width 0.2) (layer "B.Cu") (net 16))
 (segment (start 192.06 85.77) (end 198.83 79) (width 0.2) (layer "B.Cu") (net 16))
 (segment (start 163.905 61.595) (end 161.36 61.595) (width 0.2) (layer "B.Cu") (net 16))
 (segment (start 177.5 60) (end 165.5 60) (width 0.2) (layer "B.Cu") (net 16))
 (segment (start 165.5 60) (end 163.905 61.595) (width 0.2) (layer "B.Cu") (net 16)))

